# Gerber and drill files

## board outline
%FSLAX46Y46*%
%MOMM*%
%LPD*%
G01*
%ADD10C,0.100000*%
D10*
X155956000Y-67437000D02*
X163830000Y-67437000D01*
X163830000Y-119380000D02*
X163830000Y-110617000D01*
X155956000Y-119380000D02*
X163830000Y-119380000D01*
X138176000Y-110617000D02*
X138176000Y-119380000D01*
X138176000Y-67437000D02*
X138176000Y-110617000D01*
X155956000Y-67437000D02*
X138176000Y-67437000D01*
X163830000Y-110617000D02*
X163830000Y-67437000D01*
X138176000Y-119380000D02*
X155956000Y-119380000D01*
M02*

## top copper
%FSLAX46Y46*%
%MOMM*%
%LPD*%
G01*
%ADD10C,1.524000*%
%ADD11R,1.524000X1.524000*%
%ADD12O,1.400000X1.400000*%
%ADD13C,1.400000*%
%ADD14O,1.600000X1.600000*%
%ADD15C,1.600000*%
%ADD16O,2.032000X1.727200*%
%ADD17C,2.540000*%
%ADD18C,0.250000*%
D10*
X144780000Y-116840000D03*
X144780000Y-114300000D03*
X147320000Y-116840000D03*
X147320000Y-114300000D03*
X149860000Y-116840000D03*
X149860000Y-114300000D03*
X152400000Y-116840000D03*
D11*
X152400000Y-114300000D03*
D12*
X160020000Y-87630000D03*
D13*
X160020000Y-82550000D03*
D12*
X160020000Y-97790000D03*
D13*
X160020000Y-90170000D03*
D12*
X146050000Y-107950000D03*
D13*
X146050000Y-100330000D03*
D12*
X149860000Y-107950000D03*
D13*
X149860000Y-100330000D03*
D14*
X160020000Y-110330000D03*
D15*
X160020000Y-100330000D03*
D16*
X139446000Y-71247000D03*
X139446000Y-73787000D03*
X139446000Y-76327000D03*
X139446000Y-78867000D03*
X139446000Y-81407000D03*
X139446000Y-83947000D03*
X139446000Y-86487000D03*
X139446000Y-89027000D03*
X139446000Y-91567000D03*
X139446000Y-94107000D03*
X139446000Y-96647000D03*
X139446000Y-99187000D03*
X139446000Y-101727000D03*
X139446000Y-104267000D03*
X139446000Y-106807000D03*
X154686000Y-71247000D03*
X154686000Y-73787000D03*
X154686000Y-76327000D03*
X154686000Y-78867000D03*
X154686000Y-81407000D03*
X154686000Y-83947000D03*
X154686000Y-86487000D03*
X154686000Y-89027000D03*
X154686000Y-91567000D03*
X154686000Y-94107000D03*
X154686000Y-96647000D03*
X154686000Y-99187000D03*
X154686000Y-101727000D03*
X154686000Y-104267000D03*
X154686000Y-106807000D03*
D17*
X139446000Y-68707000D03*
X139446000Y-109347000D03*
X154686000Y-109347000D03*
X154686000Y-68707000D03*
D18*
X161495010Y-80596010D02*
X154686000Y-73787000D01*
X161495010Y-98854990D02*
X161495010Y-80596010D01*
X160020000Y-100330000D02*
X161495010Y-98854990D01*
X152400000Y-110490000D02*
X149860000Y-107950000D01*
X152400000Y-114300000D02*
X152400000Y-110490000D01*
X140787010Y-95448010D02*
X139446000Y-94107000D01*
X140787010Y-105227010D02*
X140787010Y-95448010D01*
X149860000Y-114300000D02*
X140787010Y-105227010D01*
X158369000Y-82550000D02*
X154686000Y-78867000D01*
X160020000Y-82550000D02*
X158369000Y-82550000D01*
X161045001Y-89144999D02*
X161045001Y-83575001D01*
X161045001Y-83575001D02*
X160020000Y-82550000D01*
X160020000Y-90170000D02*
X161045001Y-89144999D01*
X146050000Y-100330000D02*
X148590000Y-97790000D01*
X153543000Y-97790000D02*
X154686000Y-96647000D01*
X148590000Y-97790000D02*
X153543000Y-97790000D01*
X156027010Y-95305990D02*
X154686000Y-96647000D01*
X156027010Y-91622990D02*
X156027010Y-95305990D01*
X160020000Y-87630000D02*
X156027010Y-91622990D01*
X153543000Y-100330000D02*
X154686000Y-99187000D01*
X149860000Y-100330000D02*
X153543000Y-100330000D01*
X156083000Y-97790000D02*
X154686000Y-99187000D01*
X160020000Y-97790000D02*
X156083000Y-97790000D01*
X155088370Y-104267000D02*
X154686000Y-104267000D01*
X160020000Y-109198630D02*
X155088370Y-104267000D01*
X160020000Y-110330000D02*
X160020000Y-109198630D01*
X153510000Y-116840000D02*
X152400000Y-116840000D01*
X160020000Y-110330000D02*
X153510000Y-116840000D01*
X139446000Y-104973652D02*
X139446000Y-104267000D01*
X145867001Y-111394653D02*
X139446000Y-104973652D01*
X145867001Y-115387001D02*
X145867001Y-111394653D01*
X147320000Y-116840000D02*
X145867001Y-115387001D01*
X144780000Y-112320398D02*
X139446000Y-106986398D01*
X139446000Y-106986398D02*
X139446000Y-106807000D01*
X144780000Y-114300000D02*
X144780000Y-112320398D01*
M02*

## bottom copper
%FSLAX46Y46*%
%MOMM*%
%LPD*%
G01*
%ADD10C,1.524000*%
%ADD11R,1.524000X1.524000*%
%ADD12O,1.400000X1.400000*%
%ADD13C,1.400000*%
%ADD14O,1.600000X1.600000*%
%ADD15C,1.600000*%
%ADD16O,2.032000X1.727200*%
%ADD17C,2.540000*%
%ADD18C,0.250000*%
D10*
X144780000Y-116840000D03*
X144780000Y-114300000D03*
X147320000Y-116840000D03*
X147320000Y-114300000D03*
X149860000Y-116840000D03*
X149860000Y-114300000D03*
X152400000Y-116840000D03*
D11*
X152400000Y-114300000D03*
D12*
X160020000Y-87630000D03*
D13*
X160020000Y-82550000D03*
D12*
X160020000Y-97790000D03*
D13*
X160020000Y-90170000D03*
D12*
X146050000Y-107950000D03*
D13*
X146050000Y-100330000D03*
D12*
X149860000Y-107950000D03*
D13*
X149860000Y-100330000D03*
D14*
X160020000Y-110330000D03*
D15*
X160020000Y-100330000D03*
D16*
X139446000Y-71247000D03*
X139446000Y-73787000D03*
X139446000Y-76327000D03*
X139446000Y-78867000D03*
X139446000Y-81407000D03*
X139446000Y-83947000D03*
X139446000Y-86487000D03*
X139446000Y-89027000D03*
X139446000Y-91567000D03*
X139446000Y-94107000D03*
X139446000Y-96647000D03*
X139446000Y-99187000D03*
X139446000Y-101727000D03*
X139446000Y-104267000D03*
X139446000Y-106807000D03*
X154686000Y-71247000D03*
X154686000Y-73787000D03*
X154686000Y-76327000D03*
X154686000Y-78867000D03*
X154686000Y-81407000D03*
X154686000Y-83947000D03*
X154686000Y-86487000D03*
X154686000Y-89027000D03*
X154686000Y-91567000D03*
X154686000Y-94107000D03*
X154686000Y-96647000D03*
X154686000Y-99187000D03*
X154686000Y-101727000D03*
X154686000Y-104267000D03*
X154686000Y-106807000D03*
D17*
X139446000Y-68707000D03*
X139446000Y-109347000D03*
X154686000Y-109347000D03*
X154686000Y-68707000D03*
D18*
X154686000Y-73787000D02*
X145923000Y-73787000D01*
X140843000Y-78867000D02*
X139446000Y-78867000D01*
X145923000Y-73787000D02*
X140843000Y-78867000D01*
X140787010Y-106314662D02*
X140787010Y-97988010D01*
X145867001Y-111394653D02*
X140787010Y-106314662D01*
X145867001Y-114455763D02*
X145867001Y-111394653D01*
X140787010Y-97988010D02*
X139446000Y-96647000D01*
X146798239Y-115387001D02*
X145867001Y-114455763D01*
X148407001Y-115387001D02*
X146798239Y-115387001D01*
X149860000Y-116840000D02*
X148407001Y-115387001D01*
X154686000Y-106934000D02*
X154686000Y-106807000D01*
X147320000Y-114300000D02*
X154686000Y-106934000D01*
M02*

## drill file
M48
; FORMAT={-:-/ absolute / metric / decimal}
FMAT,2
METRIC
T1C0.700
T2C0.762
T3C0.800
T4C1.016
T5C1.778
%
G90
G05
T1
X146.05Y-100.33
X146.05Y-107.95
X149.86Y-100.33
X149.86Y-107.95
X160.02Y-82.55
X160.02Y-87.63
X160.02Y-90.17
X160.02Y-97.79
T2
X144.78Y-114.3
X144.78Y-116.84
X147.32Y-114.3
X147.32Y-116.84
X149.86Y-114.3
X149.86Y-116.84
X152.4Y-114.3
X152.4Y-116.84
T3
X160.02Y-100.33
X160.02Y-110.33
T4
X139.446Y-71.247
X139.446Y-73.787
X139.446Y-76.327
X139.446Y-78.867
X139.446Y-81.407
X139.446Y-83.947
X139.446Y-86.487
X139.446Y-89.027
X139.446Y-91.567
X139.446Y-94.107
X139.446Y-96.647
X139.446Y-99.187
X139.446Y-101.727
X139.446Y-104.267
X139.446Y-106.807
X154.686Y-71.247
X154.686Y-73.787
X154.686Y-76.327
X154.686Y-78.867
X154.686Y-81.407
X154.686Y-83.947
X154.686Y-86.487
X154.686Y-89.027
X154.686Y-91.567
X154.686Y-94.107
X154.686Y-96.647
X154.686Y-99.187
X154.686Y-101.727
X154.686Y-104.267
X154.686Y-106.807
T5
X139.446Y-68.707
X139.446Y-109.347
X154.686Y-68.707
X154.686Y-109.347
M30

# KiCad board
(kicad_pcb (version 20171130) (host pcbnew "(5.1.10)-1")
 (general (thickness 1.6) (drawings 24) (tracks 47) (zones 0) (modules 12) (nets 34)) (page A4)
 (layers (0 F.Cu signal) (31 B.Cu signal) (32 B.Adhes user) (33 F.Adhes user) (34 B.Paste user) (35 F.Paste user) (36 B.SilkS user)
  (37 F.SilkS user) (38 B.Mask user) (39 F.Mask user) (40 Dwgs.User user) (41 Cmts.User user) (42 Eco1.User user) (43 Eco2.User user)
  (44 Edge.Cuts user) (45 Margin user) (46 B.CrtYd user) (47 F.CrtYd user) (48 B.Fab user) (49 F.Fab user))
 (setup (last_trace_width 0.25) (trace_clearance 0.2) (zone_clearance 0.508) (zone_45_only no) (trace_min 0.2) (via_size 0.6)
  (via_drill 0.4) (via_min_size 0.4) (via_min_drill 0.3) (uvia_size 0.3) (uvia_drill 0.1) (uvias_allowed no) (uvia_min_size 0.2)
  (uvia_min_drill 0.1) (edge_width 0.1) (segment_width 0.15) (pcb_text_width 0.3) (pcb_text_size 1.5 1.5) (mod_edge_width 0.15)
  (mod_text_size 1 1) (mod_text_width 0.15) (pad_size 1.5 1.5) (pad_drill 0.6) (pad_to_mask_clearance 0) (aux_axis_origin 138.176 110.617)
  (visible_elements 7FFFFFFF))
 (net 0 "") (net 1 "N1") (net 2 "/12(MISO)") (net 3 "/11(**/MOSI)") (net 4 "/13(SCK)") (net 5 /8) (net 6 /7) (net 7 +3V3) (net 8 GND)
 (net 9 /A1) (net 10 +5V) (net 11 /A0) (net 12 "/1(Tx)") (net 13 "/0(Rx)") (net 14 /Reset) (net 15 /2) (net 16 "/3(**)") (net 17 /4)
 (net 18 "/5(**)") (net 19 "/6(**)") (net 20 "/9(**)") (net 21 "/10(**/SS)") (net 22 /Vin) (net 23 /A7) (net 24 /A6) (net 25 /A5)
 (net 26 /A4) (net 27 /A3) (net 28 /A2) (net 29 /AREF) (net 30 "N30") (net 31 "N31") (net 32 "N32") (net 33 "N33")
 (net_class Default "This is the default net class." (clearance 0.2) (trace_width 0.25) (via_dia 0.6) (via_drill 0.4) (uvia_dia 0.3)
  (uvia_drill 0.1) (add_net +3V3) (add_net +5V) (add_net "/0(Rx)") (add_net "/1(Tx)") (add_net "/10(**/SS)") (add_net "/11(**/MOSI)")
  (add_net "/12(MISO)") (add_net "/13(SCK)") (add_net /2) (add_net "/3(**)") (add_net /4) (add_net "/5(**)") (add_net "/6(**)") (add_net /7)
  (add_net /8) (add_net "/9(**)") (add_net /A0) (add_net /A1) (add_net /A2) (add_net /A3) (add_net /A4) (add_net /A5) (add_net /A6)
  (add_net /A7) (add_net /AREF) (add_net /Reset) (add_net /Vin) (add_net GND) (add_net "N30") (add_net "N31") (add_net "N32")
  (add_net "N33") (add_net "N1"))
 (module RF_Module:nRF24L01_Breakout (layer F.Cu) (at 152.4 114.3 270)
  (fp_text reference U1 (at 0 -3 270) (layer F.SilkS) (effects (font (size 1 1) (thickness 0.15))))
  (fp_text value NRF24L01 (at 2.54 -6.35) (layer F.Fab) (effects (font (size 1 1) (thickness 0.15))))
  (pad 8 thru_hole circle (at 2.54 7.62 270) (size 1.524 1.524) (drill 0.762) (layers *.Cu *.Mask) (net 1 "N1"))
  (pad 7 thru_hole circle (at 0 7.62 270) (size 1.524 1.524) (drill 0.762) (layers *.Cu *.Mask) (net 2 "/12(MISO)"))
  (pad 6 thru_hole circle (at 2.54 5.08 270) (size 1.524 1.524) (drill 0.762) (layers *.Cu *.Mask) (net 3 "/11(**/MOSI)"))
  (pad 5 thru_hole circle (at 0 5.08 270) (size 1.524 1.524) (drill 0.762) (layers *.Cu *.Mask) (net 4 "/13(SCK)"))
  (pad 4 thru_hole circle (at 2.54 2.54 270) (size 1.524 1.524) (drill 0.762) (layers *.Cu *.Mask) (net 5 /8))
  (pad 3 thru_hole circle (at 0 2.54 270) (size 1.524 1.524) (drill 0.762) (layers *.Cu *.Mask) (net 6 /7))
  (pad 2 thru_hole circle (at 2.54 0 270) (size 1.524 1.524) (drill 0.762) (layers *.Cu *.Mask) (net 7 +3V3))
  (pad 1 thru_hole rect (at 0 0 270) (size 1.524 1.524) (drill 0.762) (layers *.Cu *.Mask) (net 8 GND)))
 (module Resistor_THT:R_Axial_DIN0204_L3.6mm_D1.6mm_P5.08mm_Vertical (layer F.Cu) (at 160.02 82.55 270)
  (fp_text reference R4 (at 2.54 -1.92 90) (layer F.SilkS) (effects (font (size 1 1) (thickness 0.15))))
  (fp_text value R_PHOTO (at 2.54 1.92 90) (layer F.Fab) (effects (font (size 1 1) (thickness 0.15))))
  (pad 2 thru_hole oval (at 5.08 0 270) (size 1.4 1.4) (drill 0.7) (layers *.Cu *.Mask) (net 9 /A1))
  (pad 1 thru_hole circle (at 0 0 270) (size 1.4 1.4) (drill 0.7) (layers *.Cu *.Mask) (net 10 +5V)))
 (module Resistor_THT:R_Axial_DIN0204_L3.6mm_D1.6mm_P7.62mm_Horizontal (layer F.Cu) (at 160.02 90.17 270)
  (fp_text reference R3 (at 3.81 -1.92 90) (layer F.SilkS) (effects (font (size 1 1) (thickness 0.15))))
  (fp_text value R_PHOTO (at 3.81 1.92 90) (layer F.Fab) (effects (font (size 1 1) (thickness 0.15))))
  (pad 2 thru_hole oval (at 7.62 0 270) (size 1.4 1.4) (drill 0.7) (layers *.Cu *.Mask) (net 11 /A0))
  (pad 1 thru_hole circle (at 0 0 270) (size 1.4 1.4) (drill 0.7) (layers *.Cu *.Mask) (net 10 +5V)))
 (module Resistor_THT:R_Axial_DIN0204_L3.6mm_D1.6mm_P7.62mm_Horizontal (layer F.Cu) (at 146.05 100.33 270)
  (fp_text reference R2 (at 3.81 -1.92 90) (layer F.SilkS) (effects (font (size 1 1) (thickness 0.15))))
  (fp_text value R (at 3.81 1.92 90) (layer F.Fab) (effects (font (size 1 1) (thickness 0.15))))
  (pad 2 thru_hole oval (at 7.62 0 270) (size 1.4 1.4) (drill 0.7) (layers *.Cu *.Mask) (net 8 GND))
  (pad 1 thru_hole circle (at 0 0 270) (size 1.4 1.4) (drill 0.7) (layers *.Cu *.Mask) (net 9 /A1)))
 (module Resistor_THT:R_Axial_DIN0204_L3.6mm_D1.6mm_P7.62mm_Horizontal (layer F.Cu) (at 149.86 100.33 270)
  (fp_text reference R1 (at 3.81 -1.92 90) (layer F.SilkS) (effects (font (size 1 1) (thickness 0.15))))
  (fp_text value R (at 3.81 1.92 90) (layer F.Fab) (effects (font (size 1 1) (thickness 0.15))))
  (pad 2 thru_hole oval (at 7.62 0 270) (size 1.4 1.4) (drill 0.7) (layers *.Cu *.Mask) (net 8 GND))
  (pad 1 thru_hole circle (at 0 0 270) (size 1.4 1.4) (drill 0.7) (layers *.Cu *.Mask) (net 11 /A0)))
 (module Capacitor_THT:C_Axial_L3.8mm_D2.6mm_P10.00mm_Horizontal (layer F.Cu) (at 160.02 100.33 270)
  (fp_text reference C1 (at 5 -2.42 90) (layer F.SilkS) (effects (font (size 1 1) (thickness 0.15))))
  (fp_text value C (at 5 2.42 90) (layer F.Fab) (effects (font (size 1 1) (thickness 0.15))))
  (pad 2 thru_hole oval (at 10 0 270) (size 1.6 1.6) (drill 0.8) (layers *.Cu *.Mask) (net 7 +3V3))
  (pad 1 thru_hole circle (at 0 0 270) (size 1.6 1.6) (drill 0.8) (layers *.Cu *.Mask) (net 8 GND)))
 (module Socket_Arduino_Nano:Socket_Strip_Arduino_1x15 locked (layer F.Cu) (at 139.446 71.247 270)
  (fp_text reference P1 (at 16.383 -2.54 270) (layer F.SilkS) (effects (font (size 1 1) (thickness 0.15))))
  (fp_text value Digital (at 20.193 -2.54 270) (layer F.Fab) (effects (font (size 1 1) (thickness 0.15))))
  (pad 1 thru_hole oval (at 0 0 270) (size 1.7272 2.032) (drill 1.016) (layers *.Cu *.Mask F.SilkS) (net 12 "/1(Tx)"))
  (pad 2 thru_hole oval (at 2.54 0 270) (size 1.7272 2.032) (drill 1.016) (layers *.Cu *.Mask F.SilkS) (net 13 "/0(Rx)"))
  (pad 3 thru_hole oval (at 5.08 0 270) (size 1.7272 2.032) (drill 1.016) (layers *.Cu *.Mask F.SilkS) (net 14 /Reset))
  (pad 4 thru_hole oval (at 7.62 0 270) (size 1.7272 2.032) (drill 1.016) (layers *.Cu *.Mask F.SilkS) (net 8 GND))
  (pad 5 thru_hole oval (at 10.16 0 270) (size 1.7272 2.032) (drill 1.016) (layers *.Cu *.Mask F.SilkS) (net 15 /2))
  (pad 6 thru_hole oval (at 12.7 0 270) (size 1.7272 2.032) (drill 1.016) (layers *.Cu *.Mask F.SilkS) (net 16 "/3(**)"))
  (pad 7 thru_hole oval (at 15.24 0 270) (size 1.7272 2.032) (drill 1.016) (layers *.Cu *.Mask F.SilkS) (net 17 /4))
  (pad 8 thru_hole oval (at 17.78 0 270) (size 1.7272 2.032) (drill 1.016) (layers *.Cu *.Mask F.SilkS) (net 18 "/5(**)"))
  (pad 9 thru_hole oval (at 20.32 0 270) (size 1.7272 2.032) (drill 1.016) (layers *.Cu *.Mask F.SilkS) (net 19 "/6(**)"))
  (pad 10 thru_hole oval (at 22.86 0 270) (size 1.7272 2.032) (drill 1.016) (layers *.Cu *.Mask F.SilkS) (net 6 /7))
  (pad 11 thru_hole oval (at 25.4 0 270) (size 1.7272 2.032) (drill 1.016) (layers *.Cu *.Mask F.SilkS) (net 5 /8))
  (pad 12 thru_hole oval (at 27.94 0 270) (size 1.7272 2.032) (drill 1.016) (layers *.Cu *.Mask F.SilkS) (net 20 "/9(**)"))
  (pad 13 thru_hole oval (at 30.48 0 270) (size 1.7272 2.032) (drill 1.016) (layers *.Cu *.Mask F.SilkS) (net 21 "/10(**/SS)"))
  (pad 14 thru_hole oval (at 33.02 0 270) (size 1.7272 2.032) (drill 1.016) (layers *.Cu *.Mask F.SilkS) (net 3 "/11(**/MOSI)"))
  (pad 15 thru_hole oval (at 35.56 0 270) (size 1.7272 2.032) (drill 1.016) (layers *.Cu *.Mask F.SilkS) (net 2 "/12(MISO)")))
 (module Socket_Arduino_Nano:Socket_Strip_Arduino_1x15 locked (layer F.Cu) (at 154.686 71.247 270)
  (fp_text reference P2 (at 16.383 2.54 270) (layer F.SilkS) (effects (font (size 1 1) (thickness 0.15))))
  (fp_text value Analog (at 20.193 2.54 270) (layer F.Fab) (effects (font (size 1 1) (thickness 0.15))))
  (pad 1 thru_hole oval (at 0 0 270) (size 1.7272 2.032) (drill 1.016) (layers *.Cu *.Mask F.SilkS) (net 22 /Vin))
  (pad 2 thru_hole oval (at 2.54 0 270) (size 1.7272 2.032) (drill 1.016) (layers *.Cu *.Mask F.SilkS) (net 8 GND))
  (pad 3 thru_hole oval (at 5.08 0 270) (size 1.7272 2.032) (drill 1.016) (layers *.Cu *.Mask F.SilkS) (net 14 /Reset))
  (pad 4 thru_hole oval (at 7.62 0 270) (size 1.7272 2.032) (drill 1.016) (layers *.Cu *.Mask F.SilkS) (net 10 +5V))
  (pad 5 thru_hole oval (at 10.16 0 270) (size 1.7272 2.032) (drill 1.016) (layers *.Cu *.Mask F.SilkS) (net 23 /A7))
  (pad 6 thru_hole oval (at 12.7 0 270) (size 1.7272 2.032) (drill 1.016) (layers *.Cu *.Mask F.SilkS) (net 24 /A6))
  (pad 7 thru_hole oval (at 15.24 0 270) (size 1.7272 2.032) (drill 1.016) (layers *.Cu *.Mask F.SilkS) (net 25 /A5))
  (pad 8 thru_hole oval (at 17.78 0 270) (size 1.7272 2.032) (drill 1.016) (layers *.Cu *.Mask F.SilkS) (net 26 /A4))
  (pad 9 thru_hole oval (at 20.32 0 270) (size 1.7272 2.032) (drill 1.016) (layers *.Cu *.Mask F.SilkS) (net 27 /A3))
  (pad 10 thru_hole oval (at 22.86 0 270) (size 1.7272 2.032) (drill 1.016) (layers *.Cu *.Mask F.SilkS) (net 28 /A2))
  (pad 11 thru_hole oval (at 25.4 0 270) (size 1.7272 2.032) (drill 1.016) (layers *.Cu *.Mask F.SilkS) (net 9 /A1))
  (pad 12 thru_hole oval (at 27.94 0 270) (size 1.7272 2.032) (drill 1.016) (layers *.Cu *.Mask F.SilkS) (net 11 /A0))
  (pad 13 thru_hole oval (at 30.48 0 270) (size 1.7272 2.032) (drill 1.016) (layers *.Cu *.Mask F.SilkS) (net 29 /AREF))
  (pad 14 thru_hole oval (at 33.02 0 270) (size 1.7272 2.032) (drill 1.016) (layers *.Cu *.Mask F.SilkS) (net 7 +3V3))
  (pad 15 thru_hole oval (at 35.56 0 270) (size 1.7272 2.032) (drill 1.016) (layers *.Cu *.Mask F.SilkS) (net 4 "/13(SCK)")))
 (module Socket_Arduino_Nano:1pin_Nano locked (layer F.Cu) (at 139.446 68.707)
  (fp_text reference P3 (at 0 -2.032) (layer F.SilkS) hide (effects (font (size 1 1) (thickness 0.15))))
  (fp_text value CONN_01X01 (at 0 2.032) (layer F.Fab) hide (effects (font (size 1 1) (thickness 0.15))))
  (pad 1 thru_hole circle (at 0 0) (size 2.54 2.54) (drill 1.778) (layers *.Cu *.Mask F.SilkS) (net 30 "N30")))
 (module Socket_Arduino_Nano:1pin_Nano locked (layer F.Cu) (at 139.446 109.347)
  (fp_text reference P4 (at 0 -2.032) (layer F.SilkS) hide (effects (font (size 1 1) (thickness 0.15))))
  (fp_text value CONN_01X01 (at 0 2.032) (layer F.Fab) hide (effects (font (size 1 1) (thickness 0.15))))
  (pad 1 thru_hole circle (at 0 0) (size 2.54 2.54) (drill 1.778) (layers *.Cu *.Mask F.SilkS) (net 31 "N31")))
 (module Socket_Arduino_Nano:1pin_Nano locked (layer F.Cu) (at 154.686 109.347)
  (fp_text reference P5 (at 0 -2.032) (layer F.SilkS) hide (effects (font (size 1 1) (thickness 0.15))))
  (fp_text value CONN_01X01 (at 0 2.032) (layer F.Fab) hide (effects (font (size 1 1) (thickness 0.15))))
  (pad 1 thru_hole circle (at 0 0) (size 2.54 2.54) (drill 1.778) (layers *.Cu *.Mask F.SilkS) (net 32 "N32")))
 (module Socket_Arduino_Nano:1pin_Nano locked (layer F.Cu) (at 154.686 68.707)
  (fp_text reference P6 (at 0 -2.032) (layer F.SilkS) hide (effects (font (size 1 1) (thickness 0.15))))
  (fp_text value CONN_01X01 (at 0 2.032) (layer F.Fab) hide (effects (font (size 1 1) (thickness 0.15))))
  (pad 1 thru_hole circle (at 0 0) (size 2.54 2.54) (drill 1.778) (layers *.Cu *.Mask F.SilkS) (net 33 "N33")))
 (gr_line (start 155.956 67.437) (end 163.83 67.437) (layer Edge.Cuts) (width 0.1))
 (gr_line (start 163.83 119.38) (end 163.83 110.617) (layer Edge.Cuts) (width 0.1))
 (gr_line (start 155.956 119.38) (end 163.83 119.38) (layer Edge.Cuts) (width 0.1))
 (gr_line (start 138.176 110.617) (end 138.176 119.38) (layer Edge.Cuts) (width 0.1))
 (gr_line (start 138.176 67.437) (end 138.176 110.617) (angle 90) (layer Edge.Cuts) (width 0.1))
 (gr_line (start 155.956 67.437) (end 138.176 67.437) (angle 90) (layer Edge.Cuts) (width 0.1))
 (gr_line (start 163.83 110.617) (end 163.83 67.437) (angle 90) (layer Edge.Cuts) (width 0.1))
 (gr_line (start 138.176 119.38) (end 155.956 119.38) (angle 90) (layer Edge.Cuts) (width 0.1))
 (segment (start 161.49501 80.59601) (end 154.686 73.787) (width 0.25) (layer F.Cu) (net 8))
 (segment (start 161.49501 98.85499) (end 161.49501 80.59601) (width 0.25) (layer F.Cu) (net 8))
 (segment (start 160.02 100.33) (end 161.49501 98.85499) (width 0.25) (layer F.Cu) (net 8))
 (segment (start 152.4 110.49) (end 149.86 107.95) (width 0.25) (layer F.Cu) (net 8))
 (segment (start 152.4 114.3) (end 152.4 110.49) (width 0.25) (layer F.Cu) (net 8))
 (segment (start 154.686 73.787) (end 145.923 73.787) (width 0.25) (layer B.Cu) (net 8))
 (segment (start 140.843 78.867) (end 139.446 78.867) (width 0.25) (layer B.Cu) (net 8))
 (segment (start 145.923 73.787) (end 140.843 78.867) (width 0.25) (layer B.Cu) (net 8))
 (segment (start 140.78701 95.44801) (end 139.446 94.107) (width 0.25) (layer F.Cu) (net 6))
 (segment (start 140.78701 105.22701) (end 140.78701 95.44801) (width 0.25) (layer F.Cu) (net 6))
 (segment (start 149.86 114.3) (end 140.78701 105.22701) (width 0.25) (layer F.Cu) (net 6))
 (segment (start 140.78701 106.314662) (end 140.78701 97.98801) (width 0.25) (layer B.Cu) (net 5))
 (segment (start 145.867001 111.394653) (end 140.78701 106.314662) (width 0.25) (layer B.Cu) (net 5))
 (segment (start 145.867001 114.455763) (end 145.867001 111.394653) (width 0.25) (layer B.Cu) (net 5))
 (segment (start 140.78701 97.98801) (end 139.446 96.647) (width 0.25) (layer B.Cu) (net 5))
 (segment (start 146.798239 115.387001) (end 145.867001 114.455763) (width 0.25) (layer B.Cu) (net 5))
 (segment (start 148.407001 115.387001) (end 146.798239 115.387001) (width 0.25) (layer B.Cu) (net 5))
 (segment (start 149.86 116.84) (end 148.407001 115.387001) (width 0.25) (layer B.Cu) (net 5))
 (segment (start 158.369 82.55) (end 154.686 78.867) (width 0.25) (layer F.Cu) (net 10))
 (segment (start 160.02 82.55) (end 158.369 82.55) (width 0.25) (layer F.Cu) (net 10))
 (segment (start 161.045001 89.144999) (end 161.045001 83.575001) (width 0.25) (layer F.Cu) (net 10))
 (segment (start 161.045001 83.575001) (end 160.02 82.55) (width 0.25) (layer F.Cu) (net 10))
 (segment (start 160.02 90.17) (end 161.045001 89.144999) (width 0.25) (layer F.Cu) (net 10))
 (segment (start 146.05 100.33) (end 148.59 97.79) (width 0.25) (layer F.Cu) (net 9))
 (segment (start 153.543 97.79) (end 154.686 96.647) (width 0.25) (layer F.Cu) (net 9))
 (segment (start 148.59 97.79) (end 153.543 97.79) (width 0.25) (layer F.Cu) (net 9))
 (segment (start 156.02701 95.30599) (end 154.686 96.647) (width 0.25) (layer F.Cu) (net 9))
 (segment (start 156.02701 91.62299) (end 156.02701 95.30599) (width 0.25) (layer F.Cu) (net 9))
 (segment (start 160.02 87.63) (end 156.02701 91.62299) (width 0.25) (layer F.Cu) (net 9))
 (segment (start 153.543 100.33) (end 154.686 99.187) (width 0.25) (layer F.Cu) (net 11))
 (segment (start 149.86 100.33) (end 153.543 100.33) (width 0.25) (layer F.Cu) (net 11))
 (segment (start 156.083 97.79) (end 154.686 99.187) (width 0.25) (layer F.Cu) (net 11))
 (segment (start 160.02 97.79) (end 156.083 97.79) (width 0.25) (layer F.Cu) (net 11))
 (segment (start 154.686 106.934) (end 154.686 106.807) (width 0.25) (layer B.Cu) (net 4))
 (segment (start 147.32 114.3) (end 154.686 106.934) (width 0.25) (layer B.Cu) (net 4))
 (segment (start 155.08837 104.267) (end 154.686 104.267) (width 0.25) (layer F.Cu) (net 7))
 (segment (start 160.02 109.19863) (end 155.08837 104.267) (width 0.25) (layer F.Cu) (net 7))
 (segment (start 160.02 110.33) (end 160.02 109.19863) (width 0.25) (layer F.Cu) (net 7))
 (segment (start 153.51 116.84) (end 152.4 116.84) (width 0.25) (layer F.Cu) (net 7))
 (segment (start 160.02 110.33) (end 153.51 116.84) (width 0.25) (layer F.Cu) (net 7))
 (segment (start 139.446 104.973652) (end 139.446 104.267) (width 0.25) (layer F.Cu) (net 3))
 (segment (start 145.867001 111.394653) (end 139.446 104.973652) (width 0.25) (layer F.Cu) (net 3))
 (segment (start 145.867001 115.387001) (end 145.867001 111.394653) (width 0.25) (layer F.Cu) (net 3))
 (segment (start 147.32 116.84) (end 145.867001 115.387001) (width 0.25) (layer F.Cu) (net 3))
 (segment (start 144.78 112.320398) (end 139.446 106.986398) (width 0.25) (layer F.Cu) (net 2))
 (segment (start 139.446 106.986398) (end 139.446 106.807) (width 0.25) (layer F.Cu) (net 2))
 (segment (start 144.78 114.3) (end 144.78 112.320398) (width 0.25) (layer F.Cu) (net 2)))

